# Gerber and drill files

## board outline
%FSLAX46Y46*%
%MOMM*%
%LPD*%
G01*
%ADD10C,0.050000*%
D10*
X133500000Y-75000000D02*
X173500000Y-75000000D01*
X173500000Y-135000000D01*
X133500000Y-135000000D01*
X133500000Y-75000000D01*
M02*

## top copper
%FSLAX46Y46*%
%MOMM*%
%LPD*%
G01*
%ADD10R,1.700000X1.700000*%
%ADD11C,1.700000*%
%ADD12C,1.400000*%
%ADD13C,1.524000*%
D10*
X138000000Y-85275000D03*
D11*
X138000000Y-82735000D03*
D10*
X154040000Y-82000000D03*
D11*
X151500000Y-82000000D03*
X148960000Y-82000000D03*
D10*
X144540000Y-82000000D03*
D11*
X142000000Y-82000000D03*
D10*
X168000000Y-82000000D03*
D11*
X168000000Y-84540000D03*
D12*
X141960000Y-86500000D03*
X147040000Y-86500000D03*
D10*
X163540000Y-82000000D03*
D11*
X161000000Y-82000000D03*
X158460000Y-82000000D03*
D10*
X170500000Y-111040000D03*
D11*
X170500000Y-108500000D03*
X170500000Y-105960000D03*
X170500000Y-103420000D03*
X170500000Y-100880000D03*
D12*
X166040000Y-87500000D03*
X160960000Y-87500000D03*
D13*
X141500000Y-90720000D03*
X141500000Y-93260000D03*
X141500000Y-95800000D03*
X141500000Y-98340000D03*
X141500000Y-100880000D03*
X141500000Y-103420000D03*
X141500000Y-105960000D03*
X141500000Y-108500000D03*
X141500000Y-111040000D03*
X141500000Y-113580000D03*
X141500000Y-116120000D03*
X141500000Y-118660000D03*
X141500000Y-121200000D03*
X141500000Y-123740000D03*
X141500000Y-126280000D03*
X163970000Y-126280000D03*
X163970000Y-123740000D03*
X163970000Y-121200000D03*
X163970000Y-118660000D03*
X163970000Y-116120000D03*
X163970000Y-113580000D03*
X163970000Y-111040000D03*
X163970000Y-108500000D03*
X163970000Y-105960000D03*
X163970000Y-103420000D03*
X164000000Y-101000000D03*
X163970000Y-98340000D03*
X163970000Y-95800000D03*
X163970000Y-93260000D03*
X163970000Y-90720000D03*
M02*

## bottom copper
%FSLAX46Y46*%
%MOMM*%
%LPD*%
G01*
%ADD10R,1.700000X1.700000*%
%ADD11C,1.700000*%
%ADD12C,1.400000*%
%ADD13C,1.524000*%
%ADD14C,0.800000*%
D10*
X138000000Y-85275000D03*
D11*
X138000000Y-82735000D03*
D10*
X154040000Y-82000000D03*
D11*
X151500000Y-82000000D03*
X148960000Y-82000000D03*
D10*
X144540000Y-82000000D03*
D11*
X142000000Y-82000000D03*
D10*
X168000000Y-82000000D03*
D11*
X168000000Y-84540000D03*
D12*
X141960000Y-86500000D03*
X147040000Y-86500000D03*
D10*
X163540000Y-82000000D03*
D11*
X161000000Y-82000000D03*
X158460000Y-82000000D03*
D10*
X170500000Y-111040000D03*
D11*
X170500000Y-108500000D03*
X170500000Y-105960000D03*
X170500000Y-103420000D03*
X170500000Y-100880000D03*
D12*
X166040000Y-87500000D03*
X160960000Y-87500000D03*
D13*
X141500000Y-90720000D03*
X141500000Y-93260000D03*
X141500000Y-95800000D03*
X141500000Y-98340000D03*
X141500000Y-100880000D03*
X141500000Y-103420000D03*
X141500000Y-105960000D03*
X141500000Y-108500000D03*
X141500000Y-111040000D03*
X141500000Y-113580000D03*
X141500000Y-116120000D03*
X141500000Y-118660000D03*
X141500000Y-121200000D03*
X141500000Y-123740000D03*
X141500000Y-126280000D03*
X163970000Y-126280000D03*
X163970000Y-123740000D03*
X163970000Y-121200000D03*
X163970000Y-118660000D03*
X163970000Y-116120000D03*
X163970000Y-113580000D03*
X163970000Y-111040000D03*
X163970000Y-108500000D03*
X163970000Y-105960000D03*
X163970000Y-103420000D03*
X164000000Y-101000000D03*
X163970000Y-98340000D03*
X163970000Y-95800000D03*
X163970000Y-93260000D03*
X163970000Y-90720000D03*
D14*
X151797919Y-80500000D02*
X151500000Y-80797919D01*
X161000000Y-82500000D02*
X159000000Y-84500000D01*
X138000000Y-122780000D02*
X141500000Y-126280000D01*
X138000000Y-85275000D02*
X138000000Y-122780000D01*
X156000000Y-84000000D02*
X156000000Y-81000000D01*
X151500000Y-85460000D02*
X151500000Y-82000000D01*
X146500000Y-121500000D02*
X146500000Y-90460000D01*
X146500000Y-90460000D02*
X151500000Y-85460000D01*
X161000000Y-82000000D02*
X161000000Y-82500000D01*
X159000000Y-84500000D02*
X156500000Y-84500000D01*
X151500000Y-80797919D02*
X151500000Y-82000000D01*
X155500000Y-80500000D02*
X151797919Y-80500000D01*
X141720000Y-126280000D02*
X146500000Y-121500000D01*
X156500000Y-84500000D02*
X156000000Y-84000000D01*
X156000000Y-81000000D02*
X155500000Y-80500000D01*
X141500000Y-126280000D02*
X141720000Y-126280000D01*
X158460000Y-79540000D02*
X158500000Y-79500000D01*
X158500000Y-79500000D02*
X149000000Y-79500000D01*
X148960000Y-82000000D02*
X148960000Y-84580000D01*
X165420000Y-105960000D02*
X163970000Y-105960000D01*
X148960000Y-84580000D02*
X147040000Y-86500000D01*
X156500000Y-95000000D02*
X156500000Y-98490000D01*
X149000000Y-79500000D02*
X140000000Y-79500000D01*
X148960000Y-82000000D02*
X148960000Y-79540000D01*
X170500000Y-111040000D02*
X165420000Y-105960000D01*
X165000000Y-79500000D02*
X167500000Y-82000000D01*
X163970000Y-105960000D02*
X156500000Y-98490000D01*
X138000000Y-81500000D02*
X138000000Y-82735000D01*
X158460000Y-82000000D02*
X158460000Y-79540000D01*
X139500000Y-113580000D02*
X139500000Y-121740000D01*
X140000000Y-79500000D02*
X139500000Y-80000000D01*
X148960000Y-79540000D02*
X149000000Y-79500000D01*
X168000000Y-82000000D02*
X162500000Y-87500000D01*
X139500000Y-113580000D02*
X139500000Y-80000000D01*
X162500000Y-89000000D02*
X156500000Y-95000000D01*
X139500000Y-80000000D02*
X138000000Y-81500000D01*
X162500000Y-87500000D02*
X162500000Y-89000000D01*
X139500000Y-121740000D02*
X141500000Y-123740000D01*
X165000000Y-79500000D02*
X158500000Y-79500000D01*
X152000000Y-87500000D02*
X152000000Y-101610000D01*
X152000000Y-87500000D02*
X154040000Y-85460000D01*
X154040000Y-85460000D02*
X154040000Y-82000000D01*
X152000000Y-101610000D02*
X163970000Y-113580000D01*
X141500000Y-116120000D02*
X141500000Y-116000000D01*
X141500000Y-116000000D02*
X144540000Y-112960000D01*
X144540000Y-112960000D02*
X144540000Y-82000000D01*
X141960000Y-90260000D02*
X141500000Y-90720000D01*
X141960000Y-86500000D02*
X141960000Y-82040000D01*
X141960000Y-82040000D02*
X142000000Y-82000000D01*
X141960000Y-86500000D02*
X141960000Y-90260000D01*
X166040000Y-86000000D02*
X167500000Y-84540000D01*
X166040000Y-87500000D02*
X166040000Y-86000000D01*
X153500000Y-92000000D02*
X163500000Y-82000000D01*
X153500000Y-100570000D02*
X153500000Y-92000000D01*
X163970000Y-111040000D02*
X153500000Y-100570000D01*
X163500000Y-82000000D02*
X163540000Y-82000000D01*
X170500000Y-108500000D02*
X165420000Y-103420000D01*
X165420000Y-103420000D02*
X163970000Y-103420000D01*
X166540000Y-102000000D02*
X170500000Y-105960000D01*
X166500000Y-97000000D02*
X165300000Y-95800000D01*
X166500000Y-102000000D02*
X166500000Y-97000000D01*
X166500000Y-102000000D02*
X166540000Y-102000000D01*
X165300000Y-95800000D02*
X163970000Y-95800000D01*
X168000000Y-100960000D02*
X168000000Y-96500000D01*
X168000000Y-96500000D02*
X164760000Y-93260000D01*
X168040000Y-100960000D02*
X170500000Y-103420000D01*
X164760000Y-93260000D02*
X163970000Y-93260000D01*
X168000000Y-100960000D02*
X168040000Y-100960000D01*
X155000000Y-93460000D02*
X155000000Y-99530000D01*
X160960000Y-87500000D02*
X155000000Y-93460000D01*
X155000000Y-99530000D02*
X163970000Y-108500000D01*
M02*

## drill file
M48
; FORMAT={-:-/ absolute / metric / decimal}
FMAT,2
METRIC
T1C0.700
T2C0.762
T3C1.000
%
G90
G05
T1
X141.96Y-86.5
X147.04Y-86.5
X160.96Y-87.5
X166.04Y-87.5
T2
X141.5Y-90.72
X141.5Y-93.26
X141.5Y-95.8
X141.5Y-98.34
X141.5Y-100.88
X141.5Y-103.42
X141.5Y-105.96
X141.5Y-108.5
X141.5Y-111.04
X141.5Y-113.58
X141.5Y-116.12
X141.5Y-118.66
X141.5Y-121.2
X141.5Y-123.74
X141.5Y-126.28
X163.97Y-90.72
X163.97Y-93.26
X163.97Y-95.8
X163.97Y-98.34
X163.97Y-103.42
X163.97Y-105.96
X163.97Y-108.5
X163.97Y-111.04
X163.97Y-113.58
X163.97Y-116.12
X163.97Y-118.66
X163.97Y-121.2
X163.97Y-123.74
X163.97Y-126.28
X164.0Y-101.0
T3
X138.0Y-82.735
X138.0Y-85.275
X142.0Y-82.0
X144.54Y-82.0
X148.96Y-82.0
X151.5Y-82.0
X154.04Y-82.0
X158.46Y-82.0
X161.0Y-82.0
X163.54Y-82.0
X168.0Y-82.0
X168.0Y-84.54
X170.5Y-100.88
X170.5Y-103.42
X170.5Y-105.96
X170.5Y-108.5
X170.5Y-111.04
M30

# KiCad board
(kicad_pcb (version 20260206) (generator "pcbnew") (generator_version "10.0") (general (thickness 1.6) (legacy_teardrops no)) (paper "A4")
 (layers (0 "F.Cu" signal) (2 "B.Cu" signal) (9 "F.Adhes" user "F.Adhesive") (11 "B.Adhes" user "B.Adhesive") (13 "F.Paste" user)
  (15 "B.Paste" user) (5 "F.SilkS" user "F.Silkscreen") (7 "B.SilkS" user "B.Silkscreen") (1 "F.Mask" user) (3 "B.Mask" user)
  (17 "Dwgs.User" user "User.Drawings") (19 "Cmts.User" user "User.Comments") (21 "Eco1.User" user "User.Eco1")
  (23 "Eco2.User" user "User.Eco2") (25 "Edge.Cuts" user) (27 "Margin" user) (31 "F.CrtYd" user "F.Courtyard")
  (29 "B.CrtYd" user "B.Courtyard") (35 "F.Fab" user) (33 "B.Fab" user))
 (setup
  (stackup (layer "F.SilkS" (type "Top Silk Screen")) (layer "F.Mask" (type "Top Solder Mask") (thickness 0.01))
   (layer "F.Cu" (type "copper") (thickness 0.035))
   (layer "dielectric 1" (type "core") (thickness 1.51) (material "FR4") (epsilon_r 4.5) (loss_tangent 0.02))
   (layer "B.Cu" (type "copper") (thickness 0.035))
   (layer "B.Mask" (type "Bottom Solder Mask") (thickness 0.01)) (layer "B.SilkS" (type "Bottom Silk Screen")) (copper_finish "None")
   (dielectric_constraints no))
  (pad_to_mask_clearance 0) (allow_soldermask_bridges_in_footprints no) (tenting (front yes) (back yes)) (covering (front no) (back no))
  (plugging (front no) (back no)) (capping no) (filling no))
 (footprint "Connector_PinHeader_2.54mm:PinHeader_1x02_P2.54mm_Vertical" (layer "F.Cu") (at 138 85.275 180)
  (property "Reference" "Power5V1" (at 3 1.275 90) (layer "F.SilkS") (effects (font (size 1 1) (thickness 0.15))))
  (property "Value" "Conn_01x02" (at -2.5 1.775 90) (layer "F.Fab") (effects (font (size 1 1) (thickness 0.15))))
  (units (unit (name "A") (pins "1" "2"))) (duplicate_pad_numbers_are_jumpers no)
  (pad "1" thru_hole rect (at 0 0 180) (size 1.7 1.7) (drill 1) (layers "*.Cu" "*.Mask") (remove_unused_layers no)
   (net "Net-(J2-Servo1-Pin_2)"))
  (pad "2" thru_hole circle (at 0 2.54 180) (size 1.7 1.7) (drill 1) (layers "*.Cu" "*.Mask") (remove_unused_layers no) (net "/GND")))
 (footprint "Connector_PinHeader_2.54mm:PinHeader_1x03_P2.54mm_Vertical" (layer "F.Cu") (at 154.04 82 -90)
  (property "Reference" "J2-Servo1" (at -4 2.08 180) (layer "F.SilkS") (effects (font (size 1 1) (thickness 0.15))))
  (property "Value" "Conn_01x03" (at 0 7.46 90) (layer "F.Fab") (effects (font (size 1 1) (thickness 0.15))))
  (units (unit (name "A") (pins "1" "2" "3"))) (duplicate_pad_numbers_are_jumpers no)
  (pad "1" thru_hole rect (at 0 0 270) (size 1.7 1.7) (drill 1) (layers "*.Cu" "*.Mask") (remove_unused_layers no)
   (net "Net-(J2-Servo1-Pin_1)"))
  (pad "2" thru_hole circle (at 0 2.54 270) (size 1.7 1.7) (drill 1) (layers "*.Cu" "*.Mask") (remove_unused_layers no)
   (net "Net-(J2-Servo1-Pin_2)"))
  (pad "3" thru_hole circle (at 0 5.08 270) (size 1.7 1.7) (drill 1) (layers "*.Cu" "*.Mask") (remove_unused_layers no) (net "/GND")))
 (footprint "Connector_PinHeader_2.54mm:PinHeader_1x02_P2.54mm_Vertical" (layer "F.Cu") (at 144.54 82 -90)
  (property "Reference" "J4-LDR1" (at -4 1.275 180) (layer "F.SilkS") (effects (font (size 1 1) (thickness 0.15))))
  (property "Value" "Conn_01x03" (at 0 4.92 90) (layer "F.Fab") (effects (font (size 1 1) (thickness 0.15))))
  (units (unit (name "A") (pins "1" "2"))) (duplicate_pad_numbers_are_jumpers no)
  (pad "1" thru_hole rect (at 0 0 270) (size 1.7 1.7) (drill 1) (layers "*.Cu" "*.Mask") (remove_unused_layers no) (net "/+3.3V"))
  (pad "2" thru_hole circle (at 0 2.54 270) (size 1.7 1.7) (drill 1) (layers "*.Cu" "*.Mask") (remove_unused_layers no)
   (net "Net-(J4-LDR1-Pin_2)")))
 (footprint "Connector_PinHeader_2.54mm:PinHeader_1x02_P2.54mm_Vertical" (layer "F.Cu") (at 168 82)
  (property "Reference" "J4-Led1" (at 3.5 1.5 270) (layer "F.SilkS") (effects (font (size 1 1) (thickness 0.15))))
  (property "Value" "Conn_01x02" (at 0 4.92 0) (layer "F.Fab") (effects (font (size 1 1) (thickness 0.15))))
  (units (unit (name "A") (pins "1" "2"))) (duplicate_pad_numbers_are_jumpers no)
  (pad "1" thru_hole rect (at 0 0) (size 1.7 1.7) (drill 1) (layers "*.Cu" "*.Mask") (remove_unused_layers no) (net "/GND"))
  (pad "2" thru_hole circle (at 0 2.54) (size 1.7 1.7) (drill 1) (layers "*.Cu" "*.Mask") (remove_unused_layers no)
   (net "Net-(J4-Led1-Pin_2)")))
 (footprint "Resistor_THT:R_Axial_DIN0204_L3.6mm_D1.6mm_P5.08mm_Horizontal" (layer "F.Cu") (at 141.96 86.5)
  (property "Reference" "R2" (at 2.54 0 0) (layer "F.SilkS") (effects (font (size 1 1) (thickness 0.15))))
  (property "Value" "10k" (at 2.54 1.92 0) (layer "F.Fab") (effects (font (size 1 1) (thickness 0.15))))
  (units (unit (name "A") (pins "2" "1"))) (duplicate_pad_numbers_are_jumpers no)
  (pad "1" thru_hole circle (at 0 0) (size 1.4 1.4) (drill 0.7) (layers "*.Cu" "*.Mask") (remove_unused_layers no)
   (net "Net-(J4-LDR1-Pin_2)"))
  (pad "2" thru_hole circle (at 5.08 0) (size 1.4 1.4) (drill 0.7) (layers "*.Cu" "*.Mask") (remove_unused_layers no) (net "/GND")))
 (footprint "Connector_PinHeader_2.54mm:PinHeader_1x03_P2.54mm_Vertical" (layer "F.Cu") (at 163.54 82 -90)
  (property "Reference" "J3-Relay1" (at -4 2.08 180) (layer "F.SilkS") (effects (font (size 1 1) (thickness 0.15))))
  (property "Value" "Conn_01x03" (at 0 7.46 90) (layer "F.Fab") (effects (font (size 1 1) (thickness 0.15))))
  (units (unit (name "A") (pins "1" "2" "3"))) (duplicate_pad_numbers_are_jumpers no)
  (pad "1" thru_hole rect (at 0 0 270) (size 1.7 1.7) (drill 1) (layers "*.Cu" "*.Mask") (remove_unused_layers no)
   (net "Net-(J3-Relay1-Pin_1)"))
  (pad "2" thru_hole circle (at 0 2.54 270) (size 1.7 1.7) (drill 1) (layers "*.Cu" "*.Mask") (remove_unused_layers no)
   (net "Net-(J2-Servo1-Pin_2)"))
  (pad "3" thru_hole circle (at 0 5.08 270) (size 1.7 1.7) (drill 1) (layers "*.Cu" "*.Mask") (remove_unused_layers no) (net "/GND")))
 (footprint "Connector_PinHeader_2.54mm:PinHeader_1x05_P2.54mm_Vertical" (layer "F.Cu") (at 170.5 111.04 180)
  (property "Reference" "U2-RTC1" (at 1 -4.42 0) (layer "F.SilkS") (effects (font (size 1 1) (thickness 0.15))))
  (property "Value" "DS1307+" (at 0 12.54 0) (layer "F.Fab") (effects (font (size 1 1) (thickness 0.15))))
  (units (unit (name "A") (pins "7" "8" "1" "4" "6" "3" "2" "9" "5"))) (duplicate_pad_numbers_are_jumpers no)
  (pad "1" thru_hole rect (at 0 0 180) (size 1.7 1.7) (drill 1) (layers "*.Cu" "*.Mask") (remove_unused_layers no) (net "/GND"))
  (pad "2" thru_hole circle (at 0 2.54 180) (size 1.7 1.7) (drill 1) (layers "*.Cu" "*.Mask") (remove_unused_layers no) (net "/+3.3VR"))
  (pad "3" thru_hole circle (at 0 5.08 180) (size 1.7 1.7) (drill 1) (layers "*.Cu" "*.Mask") (remove_unused_layers no)
   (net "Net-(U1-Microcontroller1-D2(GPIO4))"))
  (pad "4" thru_hole circle (at 0 7.62 180) (size 1.7 1.7) (drill 1) (layers "*.Cu" "*.Mask") (remove_unused_layers no)
   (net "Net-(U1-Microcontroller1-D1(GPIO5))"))
  (pad "5" thru_hole circle (at 0 10.16 180) (size 1.7 1.7) (drill 1) (layers "*.Cu" "*.Mask") (remove_unused_layers no)
   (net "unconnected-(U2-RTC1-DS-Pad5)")))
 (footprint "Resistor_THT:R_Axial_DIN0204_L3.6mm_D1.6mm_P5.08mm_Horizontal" (layer "F.Cu") (at 166.04 87.5 180)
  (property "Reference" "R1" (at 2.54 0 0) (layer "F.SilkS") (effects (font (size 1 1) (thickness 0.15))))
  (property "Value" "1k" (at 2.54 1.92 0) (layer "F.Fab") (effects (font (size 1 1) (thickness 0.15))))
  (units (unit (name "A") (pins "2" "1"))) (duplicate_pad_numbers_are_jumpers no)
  (pad "1" thru_hole circle (at 0 0 180) (size 1.4 1.4) (drill 0.7) (layers "*.Cu" "*.Mask") (remove_unused_layers no)
   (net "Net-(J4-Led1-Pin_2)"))
  (pad "2" thru_hole circle (at 5.08 0 180) (size 1.4 1.4) (drill 0.7) (layers "*.Cu" "*.Mask") (remove_unused_layers no)
   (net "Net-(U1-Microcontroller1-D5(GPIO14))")))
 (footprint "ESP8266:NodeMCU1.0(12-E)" (layer "F.Cu") (at 153 108.5)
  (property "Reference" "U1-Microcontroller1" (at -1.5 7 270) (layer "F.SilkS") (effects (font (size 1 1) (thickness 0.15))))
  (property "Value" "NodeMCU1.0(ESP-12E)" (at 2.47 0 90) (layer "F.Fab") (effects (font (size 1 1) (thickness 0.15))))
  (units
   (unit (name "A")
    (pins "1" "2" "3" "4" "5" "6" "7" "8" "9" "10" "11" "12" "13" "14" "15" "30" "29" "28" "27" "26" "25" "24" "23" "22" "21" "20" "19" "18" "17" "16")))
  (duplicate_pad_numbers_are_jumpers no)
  (pad "1" thru_hole circle (at -11.5 -17.78) (size 1.524 1.524) (drill 0.762) (layers "*.Cu" "*.Mask" "F.SilkS") (remove_unused_layers no)
   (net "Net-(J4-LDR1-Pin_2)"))
  (pad "2" thru_hole circle (at -11.5 -15.24) (size 1.524 1.524) (drill 0.762) (layers "*.Cu" "*.Mask" "F.SilkS") (remove_unused_layers no)
   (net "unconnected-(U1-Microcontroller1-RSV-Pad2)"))
  (pad "3" thru_hole circle (at -11.5 -12.7) (size 1.524 1.524) (drill 0.762) (layers "*.Cu" "*.Mask" "F.SilkS") (remove_unused_layers no)
   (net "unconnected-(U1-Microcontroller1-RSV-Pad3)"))
  (pad "4" thru_hole circle (at -11.5 -10.16) (size 1.524 1.524) (drill 0.762) (layers "*.Cu" "*.Mask" "F.SilkS") (remove_unused_layers no)
   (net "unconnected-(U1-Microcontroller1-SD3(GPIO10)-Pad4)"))
  (pad "5" thru_hole circle (at -11.5 -7.62) (size 1.524 1.524) (drill 0.762) (layers "*.Cu" "*.Mask" "F.SilkS") (remove_unused_layers no)
   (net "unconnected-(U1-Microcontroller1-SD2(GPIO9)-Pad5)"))
  (pad "6" thru_hole circle (at -11.5 -5.08) (size 1.524 1.524) (drill 0.762) (layers "*.Cu" "*.Mask" "F.SilkS") (remove_unused_layers no)
   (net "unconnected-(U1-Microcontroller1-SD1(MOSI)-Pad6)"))
  (pad "7" thru_hole circle (at -11.5 -2.54) (size 1.524 1.524) (drill 0.762) (layers "*.Cu" "*.Mask" "F.SilkS") (remove_unused_layers no)
   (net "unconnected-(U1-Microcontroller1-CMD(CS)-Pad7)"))
  (pad "8" thru_hole circle (at -11.5 0) (size 1.524 1.524) (drill 0.762) (layers "*.Cu" "*.Mask" "F.SilkS") (remove_unused_layers no)
   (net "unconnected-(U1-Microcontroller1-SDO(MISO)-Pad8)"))
  (pad "9" thru_hole circle (at -11.5 2.54) (size 1.524 1.524) (drill 0.762) (layers "*.Cu" "*.Mask" "F.SilkS") (remove_unused_layers no)
   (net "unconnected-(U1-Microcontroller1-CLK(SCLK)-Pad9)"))
  (pad "10" thru_hole circle (at -11.5 5.08) (size 1.524 1.524) (drill 0.762) (layers "*.Cu" "*.Mask" "F.SilkS") (remove_unused_layers no)
   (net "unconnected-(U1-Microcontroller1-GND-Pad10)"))
  (pad "11" thru_hole circle (at -11.5 7.62) (size 1.524 1.524) (drill 0.762) (layers "*.Cu" "*.Mask" "F.SilkS") (remove_unused_layers no)
   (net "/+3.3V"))
  (pad "12" thru_hole circle (at -11.5 10.16) (size 1.524 1.524) (drill 0.762) (layers "*.Cu" "*.Mask" "F.SilkS") (remove_unused_layers no)
   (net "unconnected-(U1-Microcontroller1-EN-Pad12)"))
  (pad "13" thru_hole circle (at -11.5 12.7) (size 1.524 1.524) (drill 0.762) (layers "*.Cu" "*.Mask" "F.SilkS") (remove_unused_layers no)
   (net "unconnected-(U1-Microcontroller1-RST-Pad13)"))
  (pad "14" thru_hole circle (at -11.5 15.24) (size 1.524 1.524) (drill 0.762) (layers "*.Cu" "*.Mask" "F.SilkS") (remove_unused_layers no)
   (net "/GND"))
  (pad "15" thru_hole circle (at -11.5 17.78) (size 1.524 1.524) (drill 0.762) (layers "*.Cu" "*.Mask" "F.SilkS") (remove_unused_layers no)
   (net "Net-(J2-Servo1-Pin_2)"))
  (pad "16" thru_hole circle (at 10.97 17.78) (size 1.524 1.524) (drill 0.762) (layers "*.Cu" "*.Mask" "F.SilkS") (remove_unused_layers no)
   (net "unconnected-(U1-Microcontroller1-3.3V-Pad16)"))
  (pad "17" thru_hole circle (at 10.97 15.24) (size 1.524 1.524) (drill 0.762) (layers "*.Cu" "*.Mask" "F.SilkS") (remove_unused_layers no)
   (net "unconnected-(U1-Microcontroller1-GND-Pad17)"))
  (pad "18" thru_hole circle (at 10.97 12.7) (size 1.524 1.524) (drill 0.762) (layers "*.Cu" "*.Mask" "F.SilkS") (remove_unused_layers no)
   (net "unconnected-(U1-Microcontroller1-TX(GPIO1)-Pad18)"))
  (pad "19" thru_hole circle (at 10.97 10.16) (size 1.524 1.524) (drill 0.762) (layers "*.Cu" "*.Mask" "F.SilkS") (remove_unused_layers no)
   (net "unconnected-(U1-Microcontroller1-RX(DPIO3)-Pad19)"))
  (pad "20" thru_hole circle (at 10.97 7.62) (size 1.524 1.524) (drill 0.762) (layers "*.Cu" "*.Mask" "F.SilkS") (remove_unused_layers no)
   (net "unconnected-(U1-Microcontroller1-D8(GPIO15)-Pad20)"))
  (pad "21" thru_hole circle (at 10.97 5.08) (size 1.524 1.524) (drill 0.762) (layers "*.Cu" "*.Mask" "F.SilkS") (remove_unused_layers no)
   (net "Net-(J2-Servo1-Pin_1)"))
  (pad "22" thru_hole circle (at 10.97 2.54) (size 1.524 1.524) (drill 0.762) (layers "*.Cu" "*.Mask" "F.SilkS") (remove_unused_layers no)
   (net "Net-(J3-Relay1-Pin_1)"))
  (pad "23" thru_hole circle (at 10.97 0) (size 1.524 1.524) (drill 0.762) (layers "*.Cu" "*.Mask" "F.SilkS") (remove_unused_layers no)
   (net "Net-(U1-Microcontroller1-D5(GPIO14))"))
  (pad "24" thru_hole circle (at 10.97 -2.54) (size 1.524 1.524) (drill 0.762) (layers "*.Cu" "*.Mask" "F.SilkS") (remove_unused_layers no)
   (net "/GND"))
  (pad "25" thru_hole circle (at 10.97 -5.08) (size 1.524 1.524) (drill 0.762) (layers "*.Cu" "*.Mask" "F.SilkS") (remove_unused_layers no)
   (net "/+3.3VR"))
  (pad "26" thru_hole circle (at 11 -7.5) (size 1.524 1.524) (drill 0.762) (layers "*.Cu" "*.Mask" "F.SilkS") (remove_unused_layers no)
   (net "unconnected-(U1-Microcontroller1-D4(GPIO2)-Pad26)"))
  (pad "27" thru_hole circle (at 10.97 -10.16) (size 1.524 1.524) (drill 0.762) (layers "*.Cu" "*.Mask" "F.SilkS") (remove_unused_layers no)
   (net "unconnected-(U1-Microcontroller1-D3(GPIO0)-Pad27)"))
  (pad "28" thru_hole circle (at 10.97 -12.7) (size 1.524 1.524) (drill 0.762) (layers "*.Cu" "*.Mask" "F.SilkS") (remove_unused_layers no)
   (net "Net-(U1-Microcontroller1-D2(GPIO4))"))
  (pad "29" thru_hole circle (at 10.97 -15.24) (size 1.524 1.524) (drill 0.762) (layers "*.Cu" "*.Mask" "F.SilkS") (remove_unused_layers no)
   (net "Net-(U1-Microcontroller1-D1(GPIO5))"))
  (pad "30" thru_hole circle (at 10.97 -17.78) (size 1.524 1.524) (drill 0.762) (layers "*.Cu" "*.Mask" "F.SilkS") (remove_unused_layers no)
   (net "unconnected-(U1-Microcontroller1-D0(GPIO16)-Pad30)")))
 (gr_rect (start 133.5 75) (end 173.5 135) (stroke (width 0.05) (type solid)) (fill no) (layer "Edge.Cuts"))
 (segment (start 151.797919 80.5) (end 151.5 80.797919) (width 0.8) (layer "B.Cu") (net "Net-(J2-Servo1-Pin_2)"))
 (segment (start 161 82.5) (end 159 84.5) (width 0.8) (layer "B.Cu") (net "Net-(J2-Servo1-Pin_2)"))
 (segment (start 138 122.78) (end 141.5 126.28) (width 0.8) (layer "B.Cu") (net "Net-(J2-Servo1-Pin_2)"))
 (segment (start 138 85.275) (end 138 122.78) (width 0.8) (layer "B.Cu") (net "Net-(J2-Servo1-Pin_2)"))
 (segment (start 156 84) (end 156 81) (width 0.8) (layer "B.Cu") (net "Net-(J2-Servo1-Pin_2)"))
 (segment (start 151.5 85.46) (end 151.5 82) (width 0.8) (layer "B.Cu") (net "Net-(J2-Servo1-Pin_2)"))
 (segment (start 146.5 121.5) (end 146.5 90.46) (width 0.8) (layer "B.Cu") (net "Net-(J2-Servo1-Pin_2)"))
 (segment (start 146.5 90.46) (end 151.5 85.46) (width 0.8) (layer "B.Cu") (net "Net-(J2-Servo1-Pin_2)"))
 (segment (start 161 82) (end 161 82.5) (width 0.8) (layer "B.Cu") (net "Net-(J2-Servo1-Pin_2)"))
 (segment (start 159 84.5) (end 156.5 84.5) (width 0.8) (layer "B.Cu") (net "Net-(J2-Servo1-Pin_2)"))
 (segment (start 151.5 80.797919) (end 151.5 82) (width 0.8) (layer "B.Cu") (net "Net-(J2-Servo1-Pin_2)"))
 (segment (start 155.5 80.5) (end 151.797919 80.5) (width 0.8) (layer "B.Cu") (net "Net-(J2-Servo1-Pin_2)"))
 (segment (start 141.72 126.28) (end 146.5 121.5) (width 0.8) (layer "B.Cu") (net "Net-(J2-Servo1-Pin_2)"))
 (segment (start 156.5 84.5) (end 156 84) (width 0.8) (layer "B.Cu") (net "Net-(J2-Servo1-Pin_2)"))
 (segment (start 156 81) (end 155.5 80.5) (width 0.8) (layer "B.Cu") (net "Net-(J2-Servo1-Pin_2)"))
 (segment (start 141.5 126.28) (end 141.72 126.28) (width 0.8) (layer "B.Cu") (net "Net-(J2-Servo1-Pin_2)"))
 (segment (start 158.46 79.54) (end 158.5 79.5) (width 0.8) (layer "B.Cu") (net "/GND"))
 (segment (start 158.5 79.5) (end 149 79.5) (width 0.8) (layer "B.Cu") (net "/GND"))
 (segment (start 148.96 82) (end 148.96 84.58) (width 0.8) (layer "B.Cu") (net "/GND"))
 (segment (start 165.42 105.96) (end 163.97 105.96) (width 0.8) (layer "B.Cu") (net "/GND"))
 (segment (start 148.96 84.58) (end 147.04 86.5) (width 0.8) (layer "B.Cu") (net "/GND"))
 (segment (start 156.5 95) (end 156.5 98.49) (width 0.8) (layer "B.Cu") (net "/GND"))
 (segment (start 149 79.5) (end 140 79.5) (width 0.8) (layer "B.Cu") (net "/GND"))
 (segment (start 148.96 82) (end 148.96 79.54) (width 0.8) (layer "B.Cu") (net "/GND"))
 (segment (start 170.5 111.04) (end 165.42 105.96) (width 0.8) (layer "B.Cu") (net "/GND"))
 (segment (start 165 79.5) (end 167.5 82) (width 0.8) (layer "B.Cu") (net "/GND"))
 (segment (start 163.97 105.96) (end 156.5 98.49) (width 0.8) (layer "B.Cu") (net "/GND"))
 (segment (start 138 81.5) (end 138 82.735) (width 0.8) (layer "B.Cu") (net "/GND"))
 (segment (start 158.46 82) (end 158.46 79.54) (width 0.8) (layer "B.Cu") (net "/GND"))
 (segment (start 139.5 113.58) (end 139.5 121.74) (width 0.8) (layer "B.Cu") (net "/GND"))
 (segment (start 140 79.5) (end 139.5 80) (width 0.8) (layer "B.Cu") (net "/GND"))
 (segment (start 148.96 79.54) (end 149 79.5) (width 0.8) (layer "B.Cu") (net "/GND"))
 (segment (start 168 82) (end 162.5 87.5) (width 0.8) (layer "B.Cu") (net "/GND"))
 (segment (start 139.5 113.58) (end 139.5 80) (width 0.8) (layer "B.Cu") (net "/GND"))
 (segment (start 162.5 89) (end 156.5 95) (width 0.8) (layer "B.Cu") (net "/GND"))
 (segment (start 139.5 80) (end 138 81.5) (width 0.8) (layer "B.Cu") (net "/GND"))
 (segment (start 162.5 87.5) (end 162.5 89) (width 0.8) (layer "B.Cu") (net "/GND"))
 (segment (start 139.5 121.74) (end 141.5 123.74) (width 0.8) (layer "B.Cu") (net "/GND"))
 (segment (start 165 79.5) (end 158.5 79.5) (width 0.8) (layer "B.Cu") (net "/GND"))
 (segment (start 152 87.5) (end 152 101.61) (width 0.8) (layer "B.Cu") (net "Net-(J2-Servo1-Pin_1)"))
 (segment (start 152 87.5) (end 154.04 85.46) (width 0.8) (layer "B.Cu") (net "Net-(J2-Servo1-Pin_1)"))
 (segment (start 154.04 85.46) (end 154.04 82) (width 0.8) (layer "B.Cu") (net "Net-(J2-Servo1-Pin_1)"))
 (segment (start 152 101.61) (end 163.97 113.58) (width 0.8) (layer "B.Cu") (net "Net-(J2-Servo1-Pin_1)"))
 (segment (start 141.5 116.12) (end 141.5 116) (width 0.8) (layer "B.Cu") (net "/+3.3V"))
 (segment (start 141.5 116) (end 144.54 112.96) (width 0.8) (layer "B.Cu") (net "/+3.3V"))
 (segment (start 144.54 112.96) (end 144.54 82) (width 0.8) (layer "B.Cu") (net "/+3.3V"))
 (segment (start 141.96 90.26) (end 141.5 90.72) (width 0.8) (layer "B.Cu") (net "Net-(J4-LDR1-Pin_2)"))
 (segment (start 141.96 86.5) (end 141.96 82.04) (width 0.8) (layer "B.Cu") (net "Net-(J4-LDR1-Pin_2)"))
 (segment (start 141.96 82.04) (end 142 82) (width 0.8) (layer "B.Cu") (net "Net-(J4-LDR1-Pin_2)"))
 (segment (start 141.96 86.5) (end 141.96 90.26) (width 0.8) (layer "B.Cu") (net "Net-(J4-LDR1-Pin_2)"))
 (segment (start 166.04 86) (end 167.5 84.54) (width 0.8) (layer "B.Cu") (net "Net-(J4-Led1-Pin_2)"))
 (segment (start 166.04 87.5) (end 166.04 86) (width 0.8) (layer "B.Cu") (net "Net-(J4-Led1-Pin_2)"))
 (segment (start 153.5 92) (end 163.5 82) (width 0.8) (layer "B.Cu") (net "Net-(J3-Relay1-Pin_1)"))
 (segment (start 153.5 100.57) (end 153.5 92) (width 0.8) (layer "B.Cu") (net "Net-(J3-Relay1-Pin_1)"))
 (segment (start 163.97 111.04) (end 153.5 100.57) (width 0.8) (layer "B.Cu") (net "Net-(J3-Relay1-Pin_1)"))
 (segment (start 163.5 82) (end 163.54 82) (width 0.8) (layer "B.Cu") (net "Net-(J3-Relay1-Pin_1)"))
 (segment (start 170.5 108.5) (end 165.42 103.42) (width 0.8) (layer "B.Cu") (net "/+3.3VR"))
 (segment (start 165.42 103.42) (end 163.97 103.42) (width 0.8) (layer "B.Cu") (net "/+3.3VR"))
 (segment (start 166.54 102) (end 170.5 105.96) (width 0.8) (layer "B.Cu") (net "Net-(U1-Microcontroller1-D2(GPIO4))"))
 (segment (start 166.5 97) (end 165.3 95.8) (width 0.8) (layer "B.Cu") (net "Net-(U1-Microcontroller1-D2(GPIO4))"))
 (segment (start 166.5 102) (end 166.5 97) (width 0.8) (layer "B.Cu") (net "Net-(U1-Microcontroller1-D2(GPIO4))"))
 (segment (start 166.5 102) (end 166.54 102) (width 0.8) (layer "B.Cu") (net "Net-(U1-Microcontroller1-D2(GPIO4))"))
 (segment (start 165.3 95.8) (end 163.97 95.8) (width 0.8) (layer "B.Cu") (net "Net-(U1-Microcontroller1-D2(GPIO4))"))
 (segment (start 168 100.96) (end 168 96.5) (width 0.8) (layer "B.Cu") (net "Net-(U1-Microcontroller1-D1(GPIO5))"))
 (segment (start 168 96.5) (end 164.76 93.26) (width 0.8) (layer "B.Cu") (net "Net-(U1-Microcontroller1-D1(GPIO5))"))
 (segment (start 168.04 100.96) (end 170.5 103.42) (width 0.8) (layer "B.Cu") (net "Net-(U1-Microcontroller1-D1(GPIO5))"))
 (segment (start 164.76 93.26) (end 163.97 93.26) (width 0.8) (layer "B.Cu") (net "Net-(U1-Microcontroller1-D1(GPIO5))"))
 (segment (start 168 100.96) (end 168.04 100.96) (width 0.8) (layer "B.Cu") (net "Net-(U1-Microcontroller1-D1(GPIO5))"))
 (segment (start 155 93.46) (end 155 99.53) (width 0.8) (layer "B.Cu") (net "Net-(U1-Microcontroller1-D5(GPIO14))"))
 (segment (start 160.96 87.5) (end 155 93.46) (width 0.8) (layer "B.Cu") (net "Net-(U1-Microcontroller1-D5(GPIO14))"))
 (segment (start 155 99.53) (end 163.97 108.5) (width 0.8) (layer "B.Cu") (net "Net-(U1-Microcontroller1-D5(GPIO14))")))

